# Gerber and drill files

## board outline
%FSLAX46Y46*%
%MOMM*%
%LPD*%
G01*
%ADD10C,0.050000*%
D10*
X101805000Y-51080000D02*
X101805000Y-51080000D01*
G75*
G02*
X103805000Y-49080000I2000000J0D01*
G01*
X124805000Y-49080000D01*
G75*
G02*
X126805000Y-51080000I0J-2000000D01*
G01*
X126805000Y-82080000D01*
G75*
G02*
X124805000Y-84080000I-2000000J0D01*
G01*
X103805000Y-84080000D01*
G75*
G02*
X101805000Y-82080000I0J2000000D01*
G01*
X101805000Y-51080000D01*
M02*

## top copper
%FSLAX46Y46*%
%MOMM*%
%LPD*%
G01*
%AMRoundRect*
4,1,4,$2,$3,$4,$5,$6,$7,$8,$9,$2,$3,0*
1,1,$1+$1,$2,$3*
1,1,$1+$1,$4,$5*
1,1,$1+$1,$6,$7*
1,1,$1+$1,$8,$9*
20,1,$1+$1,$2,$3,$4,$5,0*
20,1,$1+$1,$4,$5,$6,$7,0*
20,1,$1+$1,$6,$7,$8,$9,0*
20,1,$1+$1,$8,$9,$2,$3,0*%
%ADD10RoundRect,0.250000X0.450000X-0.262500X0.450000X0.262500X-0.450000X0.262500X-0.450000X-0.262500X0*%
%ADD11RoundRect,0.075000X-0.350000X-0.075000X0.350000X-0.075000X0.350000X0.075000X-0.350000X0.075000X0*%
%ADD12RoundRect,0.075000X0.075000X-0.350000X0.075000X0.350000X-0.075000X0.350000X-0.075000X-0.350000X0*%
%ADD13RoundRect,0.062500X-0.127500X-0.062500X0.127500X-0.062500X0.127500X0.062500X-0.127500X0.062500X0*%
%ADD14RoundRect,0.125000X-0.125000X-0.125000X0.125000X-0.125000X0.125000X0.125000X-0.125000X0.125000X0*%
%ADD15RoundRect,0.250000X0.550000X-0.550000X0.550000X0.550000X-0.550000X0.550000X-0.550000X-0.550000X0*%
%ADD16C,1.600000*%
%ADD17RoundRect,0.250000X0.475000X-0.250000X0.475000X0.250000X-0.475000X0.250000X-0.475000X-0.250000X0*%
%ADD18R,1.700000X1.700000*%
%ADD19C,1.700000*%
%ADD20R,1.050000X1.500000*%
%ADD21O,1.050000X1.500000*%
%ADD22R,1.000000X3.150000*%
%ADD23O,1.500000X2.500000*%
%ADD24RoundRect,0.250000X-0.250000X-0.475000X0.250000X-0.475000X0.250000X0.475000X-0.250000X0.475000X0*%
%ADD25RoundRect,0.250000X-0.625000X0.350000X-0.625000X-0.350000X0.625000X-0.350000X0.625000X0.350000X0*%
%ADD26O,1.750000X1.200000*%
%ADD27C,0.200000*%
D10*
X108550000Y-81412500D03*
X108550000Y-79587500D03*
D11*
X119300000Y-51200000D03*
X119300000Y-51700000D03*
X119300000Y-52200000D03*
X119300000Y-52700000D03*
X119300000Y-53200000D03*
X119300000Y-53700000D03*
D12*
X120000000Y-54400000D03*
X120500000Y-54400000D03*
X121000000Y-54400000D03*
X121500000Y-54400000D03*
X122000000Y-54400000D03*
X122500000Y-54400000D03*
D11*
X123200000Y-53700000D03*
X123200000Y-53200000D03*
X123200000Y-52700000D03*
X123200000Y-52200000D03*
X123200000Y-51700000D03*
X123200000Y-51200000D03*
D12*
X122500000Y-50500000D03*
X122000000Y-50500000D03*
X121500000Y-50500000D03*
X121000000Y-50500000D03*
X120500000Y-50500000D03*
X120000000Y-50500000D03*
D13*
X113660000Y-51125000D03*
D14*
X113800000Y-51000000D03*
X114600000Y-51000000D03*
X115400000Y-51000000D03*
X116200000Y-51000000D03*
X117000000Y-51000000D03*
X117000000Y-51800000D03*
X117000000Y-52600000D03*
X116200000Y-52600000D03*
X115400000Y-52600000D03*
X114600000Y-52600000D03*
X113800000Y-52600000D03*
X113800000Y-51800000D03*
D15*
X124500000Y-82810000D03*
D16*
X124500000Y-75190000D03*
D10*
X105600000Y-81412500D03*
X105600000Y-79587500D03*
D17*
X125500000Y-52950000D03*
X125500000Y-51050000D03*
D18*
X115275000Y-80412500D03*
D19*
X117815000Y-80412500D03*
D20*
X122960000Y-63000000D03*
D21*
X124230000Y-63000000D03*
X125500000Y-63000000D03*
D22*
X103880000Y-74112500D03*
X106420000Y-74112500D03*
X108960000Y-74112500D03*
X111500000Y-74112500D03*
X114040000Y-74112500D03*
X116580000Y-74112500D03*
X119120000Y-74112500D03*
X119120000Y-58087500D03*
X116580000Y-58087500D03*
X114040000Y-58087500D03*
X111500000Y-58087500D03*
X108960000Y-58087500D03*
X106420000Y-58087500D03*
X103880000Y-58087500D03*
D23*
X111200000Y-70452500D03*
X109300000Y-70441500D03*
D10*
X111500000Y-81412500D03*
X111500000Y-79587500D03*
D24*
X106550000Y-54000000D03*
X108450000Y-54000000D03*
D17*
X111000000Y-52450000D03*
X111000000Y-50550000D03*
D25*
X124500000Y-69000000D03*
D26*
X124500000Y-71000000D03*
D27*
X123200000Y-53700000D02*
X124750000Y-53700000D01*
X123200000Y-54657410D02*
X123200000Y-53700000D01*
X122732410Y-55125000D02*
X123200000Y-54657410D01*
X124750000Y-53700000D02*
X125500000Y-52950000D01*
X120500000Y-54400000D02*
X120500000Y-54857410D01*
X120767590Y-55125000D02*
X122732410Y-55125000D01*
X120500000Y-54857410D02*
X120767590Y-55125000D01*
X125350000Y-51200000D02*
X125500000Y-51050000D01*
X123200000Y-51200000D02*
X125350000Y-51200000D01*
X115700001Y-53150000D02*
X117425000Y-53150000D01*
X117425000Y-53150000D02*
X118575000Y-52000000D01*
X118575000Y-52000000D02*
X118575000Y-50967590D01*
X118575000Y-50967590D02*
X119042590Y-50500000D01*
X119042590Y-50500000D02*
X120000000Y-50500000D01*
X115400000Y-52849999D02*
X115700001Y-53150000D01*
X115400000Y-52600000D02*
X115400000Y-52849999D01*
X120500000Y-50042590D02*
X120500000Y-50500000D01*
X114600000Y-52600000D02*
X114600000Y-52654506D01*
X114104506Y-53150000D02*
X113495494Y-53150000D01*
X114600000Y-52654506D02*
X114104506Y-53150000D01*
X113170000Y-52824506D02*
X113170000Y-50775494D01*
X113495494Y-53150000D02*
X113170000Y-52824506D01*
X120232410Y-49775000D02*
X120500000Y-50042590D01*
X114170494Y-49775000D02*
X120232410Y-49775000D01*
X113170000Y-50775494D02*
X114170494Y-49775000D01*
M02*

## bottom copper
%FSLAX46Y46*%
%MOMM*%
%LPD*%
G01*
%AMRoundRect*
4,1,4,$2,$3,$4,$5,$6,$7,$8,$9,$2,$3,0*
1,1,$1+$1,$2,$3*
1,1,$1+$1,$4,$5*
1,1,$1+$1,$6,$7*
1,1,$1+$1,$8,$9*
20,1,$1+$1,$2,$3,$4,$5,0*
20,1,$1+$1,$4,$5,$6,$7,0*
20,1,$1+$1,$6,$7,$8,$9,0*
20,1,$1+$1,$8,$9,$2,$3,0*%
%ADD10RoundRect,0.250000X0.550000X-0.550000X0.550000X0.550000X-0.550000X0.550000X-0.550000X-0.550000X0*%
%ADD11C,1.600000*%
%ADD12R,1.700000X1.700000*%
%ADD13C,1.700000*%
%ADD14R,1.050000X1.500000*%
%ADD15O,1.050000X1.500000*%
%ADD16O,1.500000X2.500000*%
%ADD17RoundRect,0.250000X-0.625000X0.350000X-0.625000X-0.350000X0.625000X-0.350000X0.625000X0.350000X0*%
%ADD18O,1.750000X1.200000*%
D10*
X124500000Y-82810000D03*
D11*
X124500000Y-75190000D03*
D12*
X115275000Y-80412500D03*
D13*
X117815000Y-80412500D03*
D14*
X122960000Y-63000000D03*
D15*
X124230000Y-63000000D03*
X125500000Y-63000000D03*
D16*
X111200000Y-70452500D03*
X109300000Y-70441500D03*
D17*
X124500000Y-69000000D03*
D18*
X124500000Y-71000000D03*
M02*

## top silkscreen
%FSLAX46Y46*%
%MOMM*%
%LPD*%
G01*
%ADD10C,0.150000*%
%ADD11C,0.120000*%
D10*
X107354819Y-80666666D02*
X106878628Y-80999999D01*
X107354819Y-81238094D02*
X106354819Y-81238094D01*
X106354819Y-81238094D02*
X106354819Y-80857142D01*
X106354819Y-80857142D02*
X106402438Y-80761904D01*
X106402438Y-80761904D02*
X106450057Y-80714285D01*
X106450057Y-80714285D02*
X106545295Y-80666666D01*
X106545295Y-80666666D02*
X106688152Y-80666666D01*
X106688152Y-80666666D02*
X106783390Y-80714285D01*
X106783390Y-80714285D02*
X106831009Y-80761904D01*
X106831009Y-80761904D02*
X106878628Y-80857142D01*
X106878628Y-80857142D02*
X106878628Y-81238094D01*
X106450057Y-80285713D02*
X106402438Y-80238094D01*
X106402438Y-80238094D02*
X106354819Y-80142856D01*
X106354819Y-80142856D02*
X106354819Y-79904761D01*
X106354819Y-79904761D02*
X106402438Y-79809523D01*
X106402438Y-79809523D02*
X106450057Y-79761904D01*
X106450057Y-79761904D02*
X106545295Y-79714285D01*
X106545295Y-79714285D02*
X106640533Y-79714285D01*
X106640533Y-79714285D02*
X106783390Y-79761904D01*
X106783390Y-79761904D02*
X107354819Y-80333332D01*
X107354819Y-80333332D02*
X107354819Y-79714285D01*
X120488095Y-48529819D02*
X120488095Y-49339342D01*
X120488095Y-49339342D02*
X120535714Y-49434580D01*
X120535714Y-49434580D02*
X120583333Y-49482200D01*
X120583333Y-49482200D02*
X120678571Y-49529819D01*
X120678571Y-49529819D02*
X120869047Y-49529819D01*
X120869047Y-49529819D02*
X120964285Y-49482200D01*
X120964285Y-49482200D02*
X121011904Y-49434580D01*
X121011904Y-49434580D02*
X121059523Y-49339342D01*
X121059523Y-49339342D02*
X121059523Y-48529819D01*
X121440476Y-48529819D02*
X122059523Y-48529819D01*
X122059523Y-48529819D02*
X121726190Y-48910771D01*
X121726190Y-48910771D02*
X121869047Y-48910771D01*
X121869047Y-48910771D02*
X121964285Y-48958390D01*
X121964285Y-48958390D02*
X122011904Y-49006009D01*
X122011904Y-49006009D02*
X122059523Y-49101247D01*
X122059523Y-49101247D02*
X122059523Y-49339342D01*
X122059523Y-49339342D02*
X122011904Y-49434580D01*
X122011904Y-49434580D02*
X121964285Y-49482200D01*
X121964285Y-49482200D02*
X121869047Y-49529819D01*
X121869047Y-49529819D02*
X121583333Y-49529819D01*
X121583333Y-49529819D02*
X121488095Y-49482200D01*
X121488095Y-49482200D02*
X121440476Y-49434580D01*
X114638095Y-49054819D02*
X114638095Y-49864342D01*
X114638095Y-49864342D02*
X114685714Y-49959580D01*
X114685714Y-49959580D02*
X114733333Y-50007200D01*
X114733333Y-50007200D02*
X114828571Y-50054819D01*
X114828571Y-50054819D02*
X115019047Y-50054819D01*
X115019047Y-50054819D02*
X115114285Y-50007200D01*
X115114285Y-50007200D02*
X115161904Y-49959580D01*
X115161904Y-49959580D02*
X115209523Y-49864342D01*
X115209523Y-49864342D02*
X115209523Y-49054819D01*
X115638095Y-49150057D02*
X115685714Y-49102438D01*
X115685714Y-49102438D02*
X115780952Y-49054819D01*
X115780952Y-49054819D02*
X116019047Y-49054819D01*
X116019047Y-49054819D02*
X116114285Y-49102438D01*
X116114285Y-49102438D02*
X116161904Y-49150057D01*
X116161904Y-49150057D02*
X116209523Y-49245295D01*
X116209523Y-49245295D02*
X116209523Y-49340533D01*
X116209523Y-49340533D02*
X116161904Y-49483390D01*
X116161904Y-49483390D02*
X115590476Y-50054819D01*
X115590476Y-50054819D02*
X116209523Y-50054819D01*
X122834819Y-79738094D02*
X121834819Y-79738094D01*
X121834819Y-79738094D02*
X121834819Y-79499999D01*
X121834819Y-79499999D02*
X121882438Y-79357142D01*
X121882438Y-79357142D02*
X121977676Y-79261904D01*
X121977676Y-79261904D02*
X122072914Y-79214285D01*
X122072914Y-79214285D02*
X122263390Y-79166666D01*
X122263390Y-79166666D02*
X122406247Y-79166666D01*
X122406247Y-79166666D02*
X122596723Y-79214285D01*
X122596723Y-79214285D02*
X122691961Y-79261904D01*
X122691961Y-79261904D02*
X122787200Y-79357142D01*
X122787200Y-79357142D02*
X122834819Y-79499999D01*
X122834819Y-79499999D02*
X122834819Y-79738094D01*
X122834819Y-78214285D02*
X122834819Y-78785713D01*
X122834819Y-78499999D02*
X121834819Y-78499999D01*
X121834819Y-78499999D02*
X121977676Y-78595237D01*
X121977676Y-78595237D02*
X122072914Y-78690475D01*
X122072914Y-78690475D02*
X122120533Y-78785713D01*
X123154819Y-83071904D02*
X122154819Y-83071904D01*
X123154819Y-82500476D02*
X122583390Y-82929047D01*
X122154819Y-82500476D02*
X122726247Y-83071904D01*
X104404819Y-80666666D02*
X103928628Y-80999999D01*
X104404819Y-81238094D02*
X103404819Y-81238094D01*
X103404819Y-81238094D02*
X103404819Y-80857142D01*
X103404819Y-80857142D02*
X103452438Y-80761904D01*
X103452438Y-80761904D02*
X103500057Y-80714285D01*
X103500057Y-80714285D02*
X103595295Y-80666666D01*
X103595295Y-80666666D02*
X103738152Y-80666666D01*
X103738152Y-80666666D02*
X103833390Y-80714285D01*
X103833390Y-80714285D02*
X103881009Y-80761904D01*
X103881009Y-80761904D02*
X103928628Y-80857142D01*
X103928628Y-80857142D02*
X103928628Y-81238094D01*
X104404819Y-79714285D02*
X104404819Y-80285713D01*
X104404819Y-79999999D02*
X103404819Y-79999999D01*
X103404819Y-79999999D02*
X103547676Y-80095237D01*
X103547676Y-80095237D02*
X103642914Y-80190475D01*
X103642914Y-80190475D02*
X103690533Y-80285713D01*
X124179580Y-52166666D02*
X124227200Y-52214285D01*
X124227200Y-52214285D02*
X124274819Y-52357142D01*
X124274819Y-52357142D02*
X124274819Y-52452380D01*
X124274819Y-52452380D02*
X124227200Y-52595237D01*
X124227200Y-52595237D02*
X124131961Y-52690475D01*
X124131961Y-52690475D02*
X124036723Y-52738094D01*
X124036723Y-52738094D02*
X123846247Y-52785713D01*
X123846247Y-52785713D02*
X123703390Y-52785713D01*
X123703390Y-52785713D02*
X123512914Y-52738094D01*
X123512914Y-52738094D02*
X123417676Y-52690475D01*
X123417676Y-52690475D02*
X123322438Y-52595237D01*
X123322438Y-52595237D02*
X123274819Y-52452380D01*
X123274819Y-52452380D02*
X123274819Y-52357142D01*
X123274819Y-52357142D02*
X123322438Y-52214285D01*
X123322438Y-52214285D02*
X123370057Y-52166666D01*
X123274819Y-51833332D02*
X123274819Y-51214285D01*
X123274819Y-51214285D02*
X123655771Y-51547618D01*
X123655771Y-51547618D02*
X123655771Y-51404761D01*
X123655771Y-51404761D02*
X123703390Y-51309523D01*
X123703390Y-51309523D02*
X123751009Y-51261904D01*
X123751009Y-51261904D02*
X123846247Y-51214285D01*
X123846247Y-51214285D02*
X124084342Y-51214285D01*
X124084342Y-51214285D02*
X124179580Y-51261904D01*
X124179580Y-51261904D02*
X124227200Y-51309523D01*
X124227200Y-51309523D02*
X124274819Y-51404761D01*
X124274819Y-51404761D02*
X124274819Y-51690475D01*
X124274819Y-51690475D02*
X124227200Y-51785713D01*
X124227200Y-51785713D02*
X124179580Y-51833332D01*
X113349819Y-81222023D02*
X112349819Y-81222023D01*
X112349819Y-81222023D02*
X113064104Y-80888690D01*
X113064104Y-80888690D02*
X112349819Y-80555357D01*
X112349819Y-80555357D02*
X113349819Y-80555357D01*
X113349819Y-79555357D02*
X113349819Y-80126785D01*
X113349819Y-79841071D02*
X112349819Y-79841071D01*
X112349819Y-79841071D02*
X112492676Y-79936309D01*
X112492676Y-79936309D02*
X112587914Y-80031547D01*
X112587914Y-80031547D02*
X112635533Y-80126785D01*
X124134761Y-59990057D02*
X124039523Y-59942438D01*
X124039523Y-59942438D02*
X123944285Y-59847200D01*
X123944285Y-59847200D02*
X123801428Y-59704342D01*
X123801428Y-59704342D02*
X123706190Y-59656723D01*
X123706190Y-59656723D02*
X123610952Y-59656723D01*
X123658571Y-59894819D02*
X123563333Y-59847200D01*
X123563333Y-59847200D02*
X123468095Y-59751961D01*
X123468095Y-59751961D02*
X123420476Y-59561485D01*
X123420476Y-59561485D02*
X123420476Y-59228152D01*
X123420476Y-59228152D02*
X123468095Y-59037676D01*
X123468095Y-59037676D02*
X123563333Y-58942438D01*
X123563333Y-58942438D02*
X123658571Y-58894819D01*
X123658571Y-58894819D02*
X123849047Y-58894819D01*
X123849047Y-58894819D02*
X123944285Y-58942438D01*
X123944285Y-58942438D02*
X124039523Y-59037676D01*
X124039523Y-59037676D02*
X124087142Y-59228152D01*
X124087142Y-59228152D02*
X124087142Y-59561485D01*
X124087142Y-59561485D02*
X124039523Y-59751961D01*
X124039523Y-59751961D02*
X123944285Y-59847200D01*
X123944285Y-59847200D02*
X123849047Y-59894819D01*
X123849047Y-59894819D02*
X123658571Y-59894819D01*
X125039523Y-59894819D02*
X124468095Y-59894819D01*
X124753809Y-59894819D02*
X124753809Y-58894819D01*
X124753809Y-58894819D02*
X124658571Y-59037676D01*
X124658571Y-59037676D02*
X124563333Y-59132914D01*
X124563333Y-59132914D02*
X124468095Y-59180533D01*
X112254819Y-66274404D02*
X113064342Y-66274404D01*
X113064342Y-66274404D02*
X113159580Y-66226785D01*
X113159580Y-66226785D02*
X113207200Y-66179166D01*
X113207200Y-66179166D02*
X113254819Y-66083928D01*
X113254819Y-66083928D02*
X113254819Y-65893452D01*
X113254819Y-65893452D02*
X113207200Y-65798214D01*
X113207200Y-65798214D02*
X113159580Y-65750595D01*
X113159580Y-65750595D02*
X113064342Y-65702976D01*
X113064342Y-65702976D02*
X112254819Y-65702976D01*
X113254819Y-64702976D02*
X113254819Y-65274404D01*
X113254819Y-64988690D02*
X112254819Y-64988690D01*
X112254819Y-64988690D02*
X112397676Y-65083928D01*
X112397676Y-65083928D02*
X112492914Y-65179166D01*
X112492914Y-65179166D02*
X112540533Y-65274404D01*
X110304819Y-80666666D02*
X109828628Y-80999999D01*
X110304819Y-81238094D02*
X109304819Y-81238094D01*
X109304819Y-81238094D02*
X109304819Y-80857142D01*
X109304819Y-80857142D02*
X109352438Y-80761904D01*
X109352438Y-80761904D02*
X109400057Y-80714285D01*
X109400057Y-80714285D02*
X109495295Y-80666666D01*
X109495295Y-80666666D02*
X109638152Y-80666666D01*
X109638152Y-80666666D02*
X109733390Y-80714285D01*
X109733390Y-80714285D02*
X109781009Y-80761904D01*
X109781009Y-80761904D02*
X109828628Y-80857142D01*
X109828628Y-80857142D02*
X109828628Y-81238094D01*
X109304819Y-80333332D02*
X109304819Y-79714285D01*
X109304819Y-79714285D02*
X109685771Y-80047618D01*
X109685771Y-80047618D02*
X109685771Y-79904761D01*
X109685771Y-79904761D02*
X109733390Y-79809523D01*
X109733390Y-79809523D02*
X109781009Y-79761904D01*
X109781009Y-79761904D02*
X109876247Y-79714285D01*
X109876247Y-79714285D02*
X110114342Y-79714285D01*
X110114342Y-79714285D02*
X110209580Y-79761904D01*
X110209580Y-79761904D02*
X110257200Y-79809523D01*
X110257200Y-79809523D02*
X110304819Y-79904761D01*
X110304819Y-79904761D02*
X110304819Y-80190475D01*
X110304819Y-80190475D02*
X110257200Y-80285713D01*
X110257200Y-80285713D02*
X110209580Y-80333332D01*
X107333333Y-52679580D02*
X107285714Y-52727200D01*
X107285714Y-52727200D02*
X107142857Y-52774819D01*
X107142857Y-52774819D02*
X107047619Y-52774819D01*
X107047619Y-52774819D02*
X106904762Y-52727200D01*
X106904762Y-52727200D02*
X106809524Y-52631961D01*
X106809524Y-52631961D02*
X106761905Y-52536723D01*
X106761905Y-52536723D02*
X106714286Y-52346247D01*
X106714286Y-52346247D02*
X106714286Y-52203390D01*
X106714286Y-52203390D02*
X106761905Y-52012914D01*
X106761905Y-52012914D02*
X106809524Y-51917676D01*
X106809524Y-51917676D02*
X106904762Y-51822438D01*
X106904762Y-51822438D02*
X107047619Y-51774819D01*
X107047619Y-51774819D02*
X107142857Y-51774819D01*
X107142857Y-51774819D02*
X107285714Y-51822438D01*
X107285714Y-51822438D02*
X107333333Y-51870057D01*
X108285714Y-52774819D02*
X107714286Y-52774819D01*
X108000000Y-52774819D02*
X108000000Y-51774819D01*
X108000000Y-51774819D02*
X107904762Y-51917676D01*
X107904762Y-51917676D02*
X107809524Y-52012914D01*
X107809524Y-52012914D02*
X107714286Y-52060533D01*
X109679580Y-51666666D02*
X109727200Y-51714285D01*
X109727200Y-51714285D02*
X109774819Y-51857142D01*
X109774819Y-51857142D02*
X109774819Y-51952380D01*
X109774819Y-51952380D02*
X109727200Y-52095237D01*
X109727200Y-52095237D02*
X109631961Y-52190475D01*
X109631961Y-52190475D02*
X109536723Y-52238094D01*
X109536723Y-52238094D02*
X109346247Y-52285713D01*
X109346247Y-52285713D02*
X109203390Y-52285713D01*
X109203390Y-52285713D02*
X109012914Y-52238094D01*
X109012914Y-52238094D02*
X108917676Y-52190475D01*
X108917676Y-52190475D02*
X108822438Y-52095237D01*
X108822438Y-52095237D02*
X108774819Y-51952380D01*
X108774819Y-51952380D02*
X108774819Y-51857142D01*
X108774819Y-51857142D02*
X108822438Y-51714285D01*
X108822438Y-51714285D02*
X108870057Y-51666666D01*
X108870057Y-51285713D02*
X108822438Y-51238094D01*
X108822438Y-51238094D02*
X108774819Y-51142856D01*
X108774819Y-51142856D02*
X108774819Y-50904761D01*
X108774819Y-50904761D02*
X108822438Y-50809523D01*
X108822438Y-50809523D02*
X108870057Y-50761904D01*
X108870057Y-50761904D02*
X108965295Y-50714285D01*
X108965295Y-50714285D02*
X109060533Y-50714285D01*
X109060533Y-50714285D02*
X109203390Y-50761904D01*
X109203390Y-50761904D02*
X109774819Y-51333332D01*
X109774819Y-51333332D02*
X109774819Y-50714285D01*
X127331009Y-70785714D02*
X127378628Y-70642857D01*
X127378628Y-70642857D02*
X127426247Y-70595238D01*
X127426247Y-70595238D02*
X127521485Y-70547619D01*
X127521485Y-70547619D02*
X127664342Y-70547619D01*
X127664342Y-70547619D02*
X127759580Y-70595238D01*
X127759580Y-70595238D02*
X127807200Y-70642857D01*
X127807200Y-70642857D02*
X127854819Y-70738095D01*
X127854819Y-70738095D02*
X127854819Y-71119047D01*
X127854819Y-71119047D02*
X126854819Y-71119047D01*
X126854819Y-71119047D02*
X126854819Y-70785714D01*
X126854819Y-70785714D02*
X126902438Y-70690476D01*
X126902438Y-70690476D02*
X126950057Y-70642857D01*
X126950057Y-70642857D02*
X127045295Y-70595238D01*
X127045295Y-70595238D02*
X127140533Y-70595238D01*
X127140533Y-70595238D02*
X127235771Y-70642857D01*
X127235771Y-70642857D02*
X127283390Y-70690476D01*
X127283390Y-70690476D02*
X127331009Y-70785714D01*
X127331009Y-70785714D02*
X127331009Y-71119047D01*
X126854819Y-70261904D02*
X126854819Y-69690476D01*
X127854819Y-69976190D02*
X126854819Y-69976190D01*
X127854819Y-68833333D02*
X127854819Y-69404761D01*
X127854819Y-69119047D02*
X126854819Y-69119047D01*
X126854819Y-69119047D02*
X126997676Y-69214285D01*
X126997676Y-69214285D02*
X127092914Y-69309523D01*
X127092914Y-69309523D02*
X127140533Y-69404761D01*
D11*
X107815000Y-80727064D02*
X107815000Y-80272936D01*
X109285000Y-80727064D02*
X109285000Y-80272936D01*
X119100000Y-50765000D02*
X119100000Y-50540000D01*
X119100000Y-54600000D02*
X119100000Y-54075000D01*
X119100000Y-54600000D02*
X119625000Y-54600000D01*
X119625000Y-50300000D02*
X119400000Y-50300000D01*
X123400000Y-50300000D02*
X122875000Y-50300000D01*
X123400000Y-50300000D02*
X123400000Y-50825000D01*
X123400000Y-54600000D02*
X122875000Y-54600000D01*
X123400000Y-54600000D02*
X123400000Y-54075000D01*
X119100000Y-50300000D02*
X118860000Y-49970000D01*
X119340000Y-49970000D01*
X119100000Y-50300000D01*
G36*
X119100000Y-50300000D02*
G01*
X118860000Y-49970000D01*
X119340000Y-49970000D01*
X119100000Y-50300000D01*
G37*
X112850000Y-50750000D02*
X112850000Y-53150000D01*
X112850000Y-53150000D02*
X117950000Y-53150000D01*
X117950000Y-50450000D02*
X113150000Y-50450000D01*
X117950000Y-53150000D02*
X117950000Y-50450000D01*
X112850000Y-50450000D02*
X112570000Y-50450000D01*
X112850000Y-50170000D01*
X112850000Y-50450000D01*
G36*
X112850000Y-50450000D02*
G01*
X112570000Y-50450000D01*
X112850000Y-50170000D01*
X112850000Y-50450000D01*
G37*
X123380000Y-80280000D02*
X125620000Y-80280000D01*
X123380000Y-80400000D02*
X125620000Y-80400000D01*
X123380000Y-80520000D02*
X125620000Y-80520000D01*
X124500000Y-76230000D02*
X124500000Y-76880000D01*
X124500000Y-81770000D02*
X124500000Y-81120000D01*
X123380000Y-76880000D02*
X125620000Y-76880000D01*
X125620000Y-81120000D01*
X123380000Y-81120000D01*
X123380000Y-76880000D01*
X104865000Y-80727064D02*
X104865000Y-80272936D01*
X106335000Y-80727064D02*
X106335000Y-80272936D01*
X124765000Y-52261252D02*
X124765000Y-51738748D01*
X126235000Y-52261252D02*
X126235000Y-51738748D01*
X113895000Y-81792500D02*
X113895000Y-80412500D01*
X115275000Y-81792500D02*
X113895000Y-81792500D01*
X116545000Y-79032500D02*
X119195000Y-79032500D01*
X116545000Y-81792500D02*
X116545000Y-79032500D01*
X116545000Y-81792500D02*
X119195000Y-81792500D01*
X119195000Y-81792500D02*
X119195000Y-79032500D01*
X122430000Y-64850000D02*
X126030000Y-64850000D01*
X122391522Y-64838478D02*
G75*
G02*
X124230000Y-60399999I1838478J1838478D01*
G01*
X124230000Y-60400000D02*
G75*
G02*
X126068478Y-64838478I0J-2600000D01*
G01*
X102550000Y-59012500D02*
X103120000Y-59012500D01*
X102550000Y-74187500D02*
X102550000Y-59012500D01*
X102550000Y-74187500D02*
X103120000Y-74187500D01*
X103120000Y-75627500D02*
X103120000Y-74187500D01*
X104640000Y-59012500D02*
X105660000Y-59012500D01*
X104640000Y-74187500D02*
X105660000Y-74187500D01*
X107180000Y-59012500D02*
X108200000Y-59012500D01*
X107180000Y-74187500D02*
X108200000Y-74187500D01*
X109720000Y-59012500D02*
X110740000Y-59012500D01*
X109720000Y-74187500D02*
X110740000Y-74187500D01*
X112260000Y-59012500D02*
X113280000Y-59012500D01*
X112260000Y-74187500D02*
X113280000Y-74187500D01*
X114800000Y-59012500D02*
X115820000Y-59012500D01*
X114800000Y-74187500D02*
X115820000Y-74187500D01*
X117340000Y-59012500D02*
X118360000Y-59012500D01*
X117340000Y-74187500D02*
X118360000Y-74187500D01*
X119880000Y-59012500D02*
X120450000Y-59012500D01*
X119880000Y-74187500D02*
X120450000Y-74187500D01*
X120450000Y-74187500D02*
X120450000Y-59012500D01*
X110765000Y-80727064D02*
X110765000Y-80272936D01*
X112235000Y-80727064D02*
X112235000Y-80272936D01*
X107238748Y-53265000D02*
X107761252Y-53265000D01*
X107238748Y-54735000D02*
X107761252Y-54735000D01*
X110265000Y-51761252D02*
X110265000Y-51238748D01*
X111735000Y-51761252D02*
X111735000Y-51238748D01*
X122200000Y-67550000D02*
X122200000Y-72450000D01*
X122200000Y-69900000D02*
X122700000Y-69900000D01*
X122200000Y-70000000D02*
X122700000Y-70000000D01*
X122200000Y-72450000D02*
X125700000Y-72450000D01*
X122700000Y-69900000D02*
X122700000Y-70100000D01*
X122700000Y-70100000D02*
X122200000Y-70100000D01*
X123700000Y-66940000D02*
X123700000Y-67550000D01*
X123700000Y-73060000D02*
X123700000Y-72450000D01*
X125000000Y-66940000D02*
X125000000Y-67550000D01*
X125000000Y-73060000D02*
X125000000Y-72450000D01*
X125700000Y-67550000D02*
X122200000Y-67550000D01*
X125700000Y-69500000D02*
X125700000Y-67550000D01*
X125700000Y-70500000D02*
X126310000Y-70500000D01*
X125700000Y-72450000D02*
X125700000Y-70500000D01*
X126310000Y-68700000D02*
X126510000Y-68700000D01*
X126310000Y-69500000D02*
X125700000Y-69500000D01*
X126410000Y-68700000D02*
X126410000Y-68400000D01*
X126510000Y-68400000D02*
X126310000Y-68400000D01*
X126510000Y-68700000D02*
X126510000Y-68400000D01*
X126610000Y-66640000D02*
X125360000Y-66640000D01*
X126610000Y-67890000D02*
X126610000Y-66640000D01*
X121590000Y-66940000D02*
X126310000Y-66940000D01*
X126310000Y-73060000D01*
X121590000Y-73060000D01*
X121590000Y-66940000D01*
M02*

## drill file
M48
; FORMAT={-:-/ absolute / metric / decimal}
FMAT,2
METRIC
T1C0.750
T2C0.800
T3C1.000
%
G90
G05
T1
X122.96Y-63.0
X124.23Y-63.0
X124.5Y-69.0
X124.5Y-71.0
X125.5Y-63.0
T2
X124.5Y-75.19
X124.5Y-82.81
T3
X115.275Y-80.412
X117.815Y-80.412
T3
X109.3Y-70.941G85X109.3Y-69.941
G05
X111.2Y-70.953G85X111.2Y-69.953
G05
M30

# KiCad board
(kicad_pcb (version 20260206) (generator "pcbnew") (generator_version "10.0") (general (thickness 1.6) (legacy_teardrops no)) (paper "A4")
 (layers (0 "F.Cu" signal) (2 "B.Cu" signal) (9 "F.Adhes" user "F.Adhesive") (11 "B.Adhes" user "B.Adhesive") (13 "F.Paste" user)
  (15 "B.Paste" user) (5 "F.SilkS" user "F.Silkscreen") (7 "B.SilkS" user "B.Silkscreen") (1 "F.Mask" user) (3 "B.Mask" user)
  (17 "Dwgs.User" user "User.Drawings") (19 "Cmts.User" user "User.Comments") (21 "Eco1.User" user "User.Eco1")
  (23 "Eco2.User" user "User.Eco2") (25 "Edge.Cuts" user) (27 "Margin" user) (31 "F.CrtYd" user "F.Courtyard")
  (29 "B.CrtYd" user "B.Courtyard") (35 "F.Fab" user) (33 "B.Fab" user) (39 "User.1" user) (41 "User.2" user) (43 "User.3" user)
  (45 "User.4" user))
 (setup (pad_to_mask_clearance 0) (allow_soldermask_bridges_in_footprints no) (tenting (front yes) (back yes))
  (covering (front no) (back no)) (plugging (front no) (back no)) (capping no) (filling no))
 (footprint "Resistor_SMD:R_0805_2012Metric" (layer "F.Cu") (at 108.55 80.5 90)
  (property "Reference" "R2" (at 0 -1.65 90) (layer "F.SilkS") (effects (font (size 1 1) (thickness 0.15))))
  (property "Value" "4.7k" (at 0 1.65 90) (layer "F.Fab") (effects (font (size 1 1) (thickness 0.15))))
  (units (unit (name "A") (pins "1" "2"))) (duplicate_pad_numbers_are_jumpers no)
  (fp_line (start -0.227064 -0.735) (end 0.227064 -0.735) (stroke (width 0.12) (type solid)) (layer "F.SilkS"))
  (fp_line (start -0.227064 0.735) (end 0.227064 0.735) (stroke (width 0.12) (type solid)) (layer "F.SilkS"))
  (pad "1" smd roundrect (at -0.9125 0 90) (size 1.025 1.4) (layers "F.Cu" "F.Mask" "F.Paste") (roundrect_rratio 0.243902) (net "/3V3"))
  (pad "2" smd roundrect (at 0.9125 0 90) (size 1.025 1.4) (layers "F.Cu" "F.Mask" "F.Paste") (roundrect_rratio 0.243902) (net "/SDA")))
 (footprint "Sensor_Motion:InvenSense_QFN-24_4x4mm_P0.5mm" (layer "F.Cu") (at 121.25 52.45)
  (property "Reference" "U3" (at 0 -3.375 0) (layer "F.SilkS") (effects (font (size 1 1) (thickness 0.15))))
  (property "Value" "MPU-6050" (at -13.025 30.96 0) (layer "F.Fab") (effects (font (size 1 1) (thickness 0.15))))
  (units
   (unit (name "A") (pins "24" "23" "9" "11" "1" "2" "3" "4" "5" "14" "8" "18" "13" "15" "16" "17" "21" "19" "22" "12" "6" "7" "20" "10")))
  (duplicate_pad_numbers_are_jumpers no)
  (fp_line (start -2.15 -1.685) (end -2.15 -1.91) (stroke (width 0.12) (type solid)) (layer "F.SilkS"))
  (fp_line (start -2.15 2.15) (end -2.15 1.625) (stroke (width 0.12) (type solid)) (layer "F.SilkS"))
  (fp_line (start -2.15 2.15) (end -1.625 2.15) (stroke (width 0.12) (type solid)) (layer "F.SilkS"))
  (fp_line (start -1.625 -2.15) (end -1.85 -2.15) (stroke (width 0.12) (type solid)) (layer "F.SilkS"))
  (fp_line (start 2.15 -2.15) (end 1.625 -2.15) (stroke (width 0.12) (type solid)) (layer "F.SilkS"))
  (fp_line (start 2.15 -2.15) (end 2.15 -1.625) (stroke (width 0.12) (type solid)) (layer "F.SilkS"))
  (fp_line (start 2.15 2.15) (end 1.625 2.15) (stroke (width 0.12) (type solid)) (layer "F.SilkS"))
  (fp_line (start 2.15 2.15) (end 2.15 1.625) (stroke (width 0.12) (type solid)) (layer "F.SilkS"))
  (fp_poly
   (pts (xy -2.15 -2.15) (xy -2.39 -2.48) (xy -1.91 -2.48) (xy -2.15 -2.15)) (stroke (width 0.12) (type solid)) (fill yes) (layer "F.SilkS"))
  (pad "1" smd roundrect (at -1.95 -1.25) (size 0.85 0.3) (layers "F.Cu" "F.Mask" "F.Paste") (roundrect_rratio 0.25)
   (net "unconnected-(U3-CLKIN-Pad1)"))
  (pad "2" smd roundrect (at -1.95 -0.75) (size 0.85 0.3) (layers "F.Cu" "F.Mask" "F.Paste") (roundrect_rratio 0.25)
   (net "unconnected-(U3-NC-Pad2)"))
  (pad "3" smd roundrect (at -1.95 -0.25) (size 0.85 0.3) (layers "F.Cu" "F.Mask" "F.Paste") (roundrect_rratio 0.25)
   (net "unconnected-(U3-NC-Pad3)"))
  (pad "4" smd roundrect (at -1.95 0.25) (size 0.85 0.3) (layers "F.Cu" "F.Mask" "F.Paste") (roundrect_rratio 0.25)
   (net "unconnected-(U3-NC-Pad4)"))
  (pad "5" smd roundrect (at -1.95 0.75) (size 0.85 0.3) (layers "F.Cu" "F.Mask" "F.Paste") (roundrect_rratio 0.25)
   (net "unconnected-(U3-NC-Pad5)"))
  (pad "6" smd roundrect (at -1.95 1.25) (size 0.85 0.3) (layers "F.Cu" "F.Mask" "F.Paste") (roundrect_rratio 0.25)
   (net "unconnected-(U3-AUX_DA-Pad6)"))
  (pad "7" smd roundrect (at -1.25 1.95 90) (size 0.85 0.3) (layers "F.Cu" "F.Mask" "F.Paste") (roundrect_rratio 0.25)
   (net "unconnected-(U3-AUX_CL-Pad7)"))
  (pad "8" smd roundrect (at -0.75 1.95 90) (size 0.85 0.3) (layers "F.Cu" "F.Mask" "F.Paste") (roundrect_rratio 0.25) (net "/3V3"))
  (pad "9" smd roundrect (at -0.25 1.95 90) (size 0.85 0.3) (layers "F.Cu" "F.Mask" "F.Paste") (roundrect_rratio 0.25) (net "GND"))
  (pad "10" smd roundrect (at 0.25 1.95 90) (size 0.85 0.3) (layers "F.Cu" "F.Mask" "F.Paste") (roundrect_rratio 0.25)
   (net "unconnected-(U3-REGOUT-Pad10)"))
  (pad "11" smd roundrect (at 0.75 1.95 90) (size 0.85 0.3) (layers "F.Cu" "F.Mask" "F.Paste") (roundrect_rratio 0.25)
   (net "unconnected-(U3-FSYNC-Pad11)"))
  (pad "12" smd roundrect (at 1.25 1.95 90) (size 0.85 0.3) (layers "F.Cu" "F.Mask" "F.Paste") (roundrect_rratio 0.25)
   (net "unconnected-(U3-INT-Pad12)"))
  (pad "13" smd roundrect (at 1.95 1.25) (size 0.85 0.3) (layers "F.Cu" "F.Mask" "F.Paste") (roundrect_rratio 0.25) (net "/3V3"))
  (pad "14" smd roundrect (at 1.95 0.75) (size 0.85 0.3) (layers "F.Cu" "F.Mask" "F.Paste") (roundrect_rratio 0.25)
   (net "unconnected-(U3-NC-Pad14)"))
  (pad "15" smd roundrect (at 1.95 0.25) (size 0.85 0.3) (layers "F.Cu" "F.Mask" "F.Paste") (roundrect_rratio 0.25)
   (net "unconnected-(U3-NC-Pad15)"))
  (pad "16" smd roundrect (at 1.95 -0.25) (size 0.85 0.3) (layers "F.Cu" "F.Mask" "F.Paste") (roundrect_rratio 0.25)
   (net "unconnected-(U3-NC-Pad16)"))
  (pad "17" smd roundrect (at 1.95 -0.75) (size 0.85 0.3) (layers "F.Cu" "F.Mask" "F.Paste") (roundrect_rratio 0.25)
   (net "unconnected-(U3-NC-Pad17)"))
  (pad "18" smd roundrect (at 1.95 -1.25) (size 0.85 0.3) (layers "F.Cu" "F.Mask" "F.Paste") (roundrect_rratio 0.25) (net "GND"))
  (pad "19" smd roundrect (at 1.25 -1.95 90) (size 0.85 0.3) (layers "F.Cu" "F.Mask" "F.Paste") (roundrect_rratio 0.25)
   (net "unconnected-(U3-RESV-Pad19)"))
  (pad "20" smd roundrect (at 0.75 -1.95 90) (size 0.85 0.3) (layers "F.Cu" "F.Mask" "F.Paste") (roundrect_rratio 0.25)
   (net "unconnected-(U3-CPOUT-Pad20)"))
  (pad "21" smd roundrect (at 0.25 -1.95 90) (size 0.85 0.3) (layers "F.Cu" "F.Mask" "F.Paste") (roundrect_rratio 0.25)
   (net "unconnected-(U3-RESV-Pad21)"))
  (pad "22" smd roundrect (at -0.25 -1.95 90) (size 0.85 0.3) (layers "F.Cu" "F.Mask" "F.Paste") (roundrect_rratio 0.25)
   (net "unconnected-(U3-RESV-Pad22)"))
  (pad "23" smd roundrect (at -0.75 -1.95 90) (size 0.85 0.3) (layers "F.Cu" "F.Mask" "F.Paste") (roundrect_rratio 0.25) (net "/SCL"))
  (pad "24" smd roundrect (at -1.25 -1.95 90) (size 0.85 0.3) (layers "F.Cu" "F.Mask" "F.Paste") (roundrect_rratio 0.25) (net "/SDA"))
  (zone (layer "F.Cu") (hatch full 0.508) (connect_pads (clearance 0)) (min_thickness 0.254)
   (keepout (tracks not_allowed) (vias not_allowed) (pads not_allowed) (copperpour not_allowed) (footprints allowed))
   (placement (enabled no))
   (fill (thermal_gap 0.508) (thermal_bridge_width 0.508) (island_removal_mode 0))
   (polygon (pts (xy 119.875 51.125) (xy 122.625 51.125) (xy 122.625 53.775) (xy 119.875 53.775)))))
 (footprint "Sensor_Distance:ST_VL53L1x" (layer "F.Cu") (at 115.4 51.8)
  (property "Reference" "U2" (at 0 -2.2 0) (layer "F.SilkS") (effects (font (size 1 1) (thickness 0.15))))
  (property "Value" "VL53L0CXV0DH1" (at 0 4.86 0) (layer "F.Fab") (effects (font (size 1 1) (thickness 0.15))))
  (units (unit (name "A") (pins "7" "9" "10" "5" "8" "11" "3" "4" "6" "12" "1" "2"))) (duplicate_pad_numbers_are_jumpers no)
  (fp_line (start -2.55 -1.05) (end -2.55 1.35) (stroke (width 0.12) (type solid)) (layer "F.SilkS"))
  (fp_line (start -2.55 1.35) (end 2.55 1.35) (stroke (width 0.12) (type solid)) (layer "F.SilkS"))
  (fp_line (start 2.55 -1.35) (end -2.25 -1.35) (stroke (width 0.12) (type solid)) (layer "F.SilkS"))
  (fp_line (start 2.55 1.35) (end 2.55 -1.35) (stroke (width 0.12) (type solid)) (layer "F.SilkS"))
  (fp_poly
   (pts (xy -2.55 -1.35) (xy -2.83 -1.35) (xy -2.55 -1.63) (xy -2.55 -1.35)) (stroke (width 0.12) (type solid)) (fill yes) (layer "F.SilkS"))
  (pad "1" smd roundrect (at -1.74 -0.675) (size 0.38 0.25) (layers "F.Cu" "F.Mask" "F.Paste") (roundrect_rratio 0.25) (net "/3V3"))
  (pad "1" smd roundrect (at -1.6 -0.8) (size 0.5 0.5) (layers "F.Cu" "F.Mask" "F.Paste") (roundrect_rratio 0.25) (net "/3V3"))
  (pad "2" smd roundrect (at -0.8 -0.8) (size 0.5 0.5) (layers "F.Cu" "F.Mask" "F.Paste") (roundrect_rratio 0.25) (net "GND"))
  (pad "3" smd roundrect (at 0 -0.8) (size 0.5 0.5) (layers "F.Cu" "F.Mask" "F.Paste") (roundrect_rratio 0.25) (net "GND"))
  (pad "4" smd roundrect (at 0.8 -0.8) (size 0.5 0.5) (layers "F.Cu" "F.Mask" "F.Paste") (roundrect_rratio 0.25) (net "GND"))
  (pad "5" smd roundrect (at 1.6 -0.8) (size 0.5 0.5) (layers "F.Cu" "F.Mask" "F.Paste") (roundrect_rratio 0.25) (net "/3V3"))
  (pad "6" smd roundrect (at 1.6 0) (size 0.5 0.5) (layers "F.Cu" "F.Mask" "F.Paste") (roundrect_rratio 0.25) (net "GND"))
  (pad "7" smd roundrect (at 1.6 0.8) (size 0.5 0.5) (layers "F.Cu" "F.Mask" "F.Paste") (roundrect_rratio 0.25)
   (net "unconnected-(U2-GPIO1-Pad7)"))
  (pad "8" smd roundrect (at 0.8 0.8) (size 0.5 0.5) (layers "F.Cu" "F.Mask" "F.Paste") (roundrect_rratio 0.25)
   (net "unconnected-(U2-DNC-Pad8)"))
  (pad "9" smd roundrect (at 0 0.8) (size 0.5 0.5) (layers "F.Cu" "F.Mask" "F.Paste") (roundrect_rratio 0.25) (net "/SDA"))
  (pad "10" smd roundrect (at -0.8 0.8) (size 0.5 0.5) (layers "F.Cu" "F.Mask" "F.Paste") (roundrect_rratio 0.25) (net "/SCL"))
  (pad "11" smd roundrect (at -1.6 0.8) (size 0.5 0.5) (layers "F.Cu" "F.Mask" "F.Paste") (roundrect_rratio 0.25) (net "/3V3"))
  (pad "12" smd roundrect (at -1.6 0) (size 0.5 0.5) (layers "F.Cu" "F.Mask" "F.Paste") (roundrect_rratio 0.25) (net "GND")))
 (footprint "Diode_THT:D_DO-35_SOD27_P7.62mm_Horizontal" (layer "F.Cu") (at 124.5 82.81 90)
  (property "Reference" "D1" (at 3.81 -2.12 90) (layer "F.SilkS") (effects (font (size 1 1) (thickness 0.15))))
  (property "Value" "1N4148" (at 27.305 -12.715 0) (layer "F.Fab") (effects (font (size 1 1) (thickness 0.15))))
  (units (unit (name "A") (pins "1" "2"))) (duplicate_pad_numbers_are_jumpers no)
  (fp_line (start 2.53 -1.12) (end 2.53 1.12) (stroke (width 0.12) (type solid)) (layer "F.SilkS"))
  (fp_line (start 2.41 -1.12) (end 2.41 1.12) (stroke (width 0.12) (type solid)) (layer "F.SilkS"))
  (fp_line (start 2.29 -1.12) (end 2.29 1.12) (stroke (width 0.12) (type solid)) (layer "F.SilkS"))
  (fp_line (start 6.58 0) (end 5.93 0) (stroke (width 0.12) (type solid)) (layer "F.SilkS"))
  (fp_line (start 1.04 0) (end 1.69 0) (stroke (width 0.12) (type solid)) (layer "F.SilkS"))
  (fp_rect (start 1.69 -1.12) (end 5.93 1.12) (stroke (width 0.12) (type solid)) (fill no) (layer "F.SilkS"))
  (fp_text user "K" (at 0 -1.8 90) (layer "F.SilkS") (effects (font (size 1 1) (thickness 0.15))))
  (pad "1" thru_hole roundrect (at 0 0 90) (size 1.6 1.6) (drill 0.8) (layers "*.Cu" "*.Mask") (remove_unused_layers no)
   (roundrect_rratio 0.15625) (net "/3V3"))
  (pad "2" thru_hole circle (at 7.62 0 90) (size 1.6 1.6) (drill 0.8) (layers "*.Cu" "*.Mask") (remove_unused_layers no) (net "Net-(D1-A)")))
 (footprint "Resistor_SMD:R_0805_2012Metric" (layer "F.Cu") (at 105.6 80.5 90)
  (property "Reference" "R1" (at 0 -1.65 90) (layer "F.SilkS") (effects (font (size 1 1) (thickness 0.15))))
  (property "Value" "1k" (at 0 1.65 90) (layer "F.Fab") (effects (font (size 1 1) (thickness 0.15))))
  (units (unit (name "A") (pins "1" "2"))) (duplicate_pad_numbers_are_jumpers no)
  (fp_line (start -0.227064 -0.735) (end 0.227064 -0.735) (stroke (width 0.12) (type solid)) (layer "F.SilkS"))
  (fp_line (start -0.227064 0.735) (end 0.227064 0.735) (stroke (width 0.12) (type solid)) (layer "F.SilkS"))
  (pad "1" smd roundrect (at -0.9125 0 90) (size 1.025 1.4) (layers "F.Cu" "F.Mask" "F.Paste") (roundrect_rratio 0.243902)
   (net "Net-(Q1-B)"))
  (pad "2" smd roundrect (at 0.9125 0 90) (size 1.025 1.4) (layers "F.Cu" "F.Mask" "F.Paste") (roundrect_rratio 0.243902)
   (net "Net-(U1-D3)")))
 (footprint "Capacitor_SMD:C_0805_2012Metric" (layer "F.Cu") (at 125.5 52 90)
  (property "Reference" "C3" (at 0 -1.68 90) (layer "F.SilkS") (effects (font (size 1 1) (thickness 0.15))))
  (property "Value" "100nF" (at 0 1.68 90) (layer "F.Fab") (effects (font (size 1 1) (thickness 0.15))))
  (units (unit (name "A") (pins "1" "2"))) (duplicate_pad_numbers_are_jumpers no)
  (fp_line (start -0.261252 -0.735) (end 0.261252 -0.735) (stroke (width 0.12) (type solid)) (layer "F.SilkS"))
  (fp_line (start -0.261252 0.735) (end 0.261252 0.735) (stroke (width 0.12) (type solid)) (layer "F.SilkS"))
  (pad "1" smd roundrect (at -0.95 0 90) (size 1 1.45) (layers "F.Cu" "F.Mask" "F.Paste") (roundrect_rratio 0.25) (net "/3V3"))
  (pad "2" smd roundrect (at 0.95 0 90) (size 1 1.45) (layers "F.Cu" "F.Mask" "F.Paste") (roundrect_rratio 0.25) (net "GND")))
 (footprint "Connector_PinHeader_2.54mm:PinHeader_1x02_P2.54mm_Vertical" (layer "F.Cu") (at 115.275 80.4125 90)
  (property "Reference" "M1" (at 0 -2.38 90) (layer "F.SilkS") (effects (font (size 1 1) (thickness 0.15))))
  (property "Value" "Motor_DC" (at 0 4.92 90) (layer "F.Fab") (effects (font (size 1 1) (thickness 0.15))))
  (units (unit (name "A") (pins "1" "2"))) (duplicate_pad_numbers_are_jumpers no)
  (fp_line (start -1.38 -1.38) (end 0 -1.38) (stroke (width 0.12) (type solid)) (layer "F.SilkS"))
  (fp_line (start -1.38 0) (end -1.38 -1.38) (stroke (width 0.12) (type solid)) (layer "F.SilkS"))
  (fp_line (start 1.38 1.27) (end 1.38 3.92) (stroke (width 0.12) (type solid)) (layer "F.SilkS"))
  (fp_line (start -1.38 1.27) (end 1.38 1.27) (stroke (width 0.12) (type solid)) (layer "F.SilkS"))
  (fp_line (start -1.38 1.27) (end -1.38 3.92) (stroke (width 0.12) (type solid)) (layer "F.SilkS"))
  (fp_line (start -1.38 3.92) (end 1.38 3.92) (stroke (width 0.12) (type solid)) (layer "F.SilkS"))
  (pad "1" thru_hole rect (at 0 0 90) (size 1.7 1.7) (drill 1) (layers "*.Cu" "*.Mask") (remove_unused_layers no) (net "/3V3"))
  (pad "2" thru_hole circle (at 0 2.54 90) (size 1.7 1.7) (drill 1) (layers "*.Cu" "*.Mask") (remove_unused_layers no) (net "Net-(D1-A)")))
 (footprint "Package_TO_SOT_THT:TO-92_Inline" (layer "F.Cu") (at 122.96 63)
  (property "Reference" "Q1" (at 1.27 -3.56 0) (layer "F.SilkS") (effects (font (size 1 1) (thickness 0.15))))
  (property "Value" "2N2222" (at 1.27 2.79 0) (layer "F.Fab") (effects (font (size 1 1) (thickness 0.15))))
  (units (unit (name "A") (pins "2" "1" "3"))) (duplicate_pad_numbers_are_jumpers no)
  (fp_line (start -0.53 1.85) (end 3.07 1.85) (stroke (width 0.12) (type solid)) (layer "F.SilkS"))
  (fp_arc (start -0.568478 1.838478) (mid -1.132087 -0.994977) (end 1.27 -2.6) (stroke (width 0.12) (type solid)) (layer "F.SilkS"))
  (fp_arc (start 1.27 -2.6) (mid 3.672087 -0.994977) (end 3.108478 1.838478) (stroke (width 0.12) (type solid)) (layer "F.SilkS"))
  (pad "1" thru_hole rect (at 0 0) (size 1.05 1.5) (drill 0.75) (layers "*.Cu" "*.Mask") (remove_unused_layers no) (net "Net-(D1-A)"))
  (pad "2" thru_hole oval (at 1.27 0) (size 1.05 1.5) (drill 0.75) (layers "*.Cu" "*.Mask") (remove_unused_layers no) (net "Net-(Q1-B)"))
  (pad "3" thru_hole oval (at 2.54 0) (size 1.05 1.5) (drill 0.75) (layers "*.Cu" "*.Mask") (remove_unused_layers no) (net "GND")))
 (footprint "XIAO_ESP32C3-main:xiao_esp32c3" (layer "F.Cu") (at 113.3 65.5125 90)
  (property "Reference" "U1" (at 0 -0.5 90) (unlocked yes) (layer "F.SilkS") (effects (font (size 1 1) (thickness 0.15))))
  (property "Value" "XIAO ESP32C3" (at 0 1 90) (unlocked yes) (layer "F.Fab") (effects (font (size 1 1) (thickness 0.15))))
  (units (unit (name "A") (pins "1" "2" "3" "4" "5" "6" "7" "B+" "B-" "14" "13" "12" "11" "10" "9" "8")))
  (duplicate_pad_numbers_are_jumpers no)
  (fp_line (start 6.5 -10.75) (end 6.5 -10.18) (stroke (width 0.12) (type solid)) (layer "F.SilkS"))
  (fp_line (start -8.675 -10.75) (end 6.5 -10.75) (stroke (width 0.12) (type solid)) (layer "F.SilkS"))
  (fp_line (start -8.675 -10.75) (end -8.675 -10.18) (stroke (width 0.12) (type solid)) (layer "F.SilkS"))
  (fp_line (start -10.115 -10.18) (end -8.675 -10.18) (stroke (width 0.12) (type solid)) (layer "F.SilkS"))
  (fp_line (start 6.5 -8.66) (end 6.5 -7.64) (stroke (width 0.12) (type solid)) (layer "F.SilkS"))
  (fp_line (start -8.675 -8.66) (end -8.675 -7.64) (stroke (width 0.12) (type solid)) (layer "F.SilkS"))
  (fp_line (start 6.5 -6.12) (end 6.5 -5.1) (stroke (width 0.12) (type solid)) (layer "F.SilkS"))
  (fp_line (start -8.675 -6.12) (end -8.675 -5.1) (stroke (width 0.12) (type solid)) (layer "F.SilkS"))
  (fp_line (start 6.5 -3.58) (end 6.5 -2.56) (stroke (width 0.12) (type solid)) (layer "F.SilkS"))
  (fp_line (start -8.675 -3.58) (end -8.675 -2.56) (stroke (width 0.12) (type solid)) (layer "F.SilkS"))
  (fp_line (start 6.5 -1.04) (end 6.5 -0.02) (stroke (width 0.12) (type solid)) (layer "F.SilkS"))
  (fp_line (start -8.675 -1.04) (end -8.675 -0.02) (stroke (width 0.12) (type solid)) (layer "F.SilkS"))
  (fp_line (start 6.5 1.5) (end 6.5 2.52) (stroke (width 0.12) (type solid)) (layer "F.SilkS"))
  (fp_line (start -8.675 1.5) (end -8.675 2.52) (stroke (width 0.12) (type solid)) (layer "F.SilkS"))
  (fp_line (start 6.5 4.04) (end 6.5 5.06) (stroke (width 0.12) (type solid)) (layer "F.SilkS"))
  (fp_line (start -8.675 4.04) (end -8.675 5.06) (stroke (width 0.12) (type solid)) (layer "F.SilkS"))
  (fp_line (start 6.5 6.58) (end 6.5 7.15) (stroke (width 0.12) (type solid)) (layer "F.SilkS"))
  (fp_line (start -8.675 6.58) (end -8.675 7.15) (stroke (width 0.12) (type solid)) (layer "F.SilkS"))
  (fp_line (start -8.675 7.15) (end 6.5 7.15) (stroke (width 0.12) (type solid)) (layer "F.SilkS"))
  (pad "1" smd rect (at -8.6 -9.42 90) (size 3.15 1) (layers "F.Cu" "F.Mask" "F.Paste") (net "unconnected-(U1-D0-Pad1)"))
  (pad "2" smd rect (at -8.6 -6.88 90) (size 3.15 1) (layers "F.Cu" "F.Mask" "F.Paste") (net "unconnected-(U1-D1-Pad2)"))
  (pad "3" smd rect (at -8.6 -4.34 90) (size 3.15 1) (layers "F.Cu" "F.Mask" "F.Paste") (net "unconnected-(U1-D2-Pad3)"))
  (pad "4" smd rect (at -8.6 -1.8 90) (size 3.15 1) (layers "F.Cu" "F.Mask" "F.Paste") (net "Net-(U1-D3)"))
  (pad "5" smd rect (at -8.6 0.74 90) (size 3.15 1) (layers "F.Cu" "F.Mask" "F.Paste") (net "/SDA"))
  (pad "6" smd rect (at -8.6 3.28 90) (size 3.15 1) (layers "F.Cu" "F.Mask" "F.Paste") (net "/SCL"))
  (pad "7" smd rect (at -8.6 5.82 90) (size 3.15 1) (layers "F.Cu" "F.Mask" "F.Paste") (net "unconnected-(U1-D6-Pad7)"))
  (pad "8" smd rect (at 7.425 5.82 90) (size 3.15 1) (layers "F.Cu" "F.Mask" "F.Paste") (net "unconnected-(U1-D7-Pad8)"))
  (pad "9" smd rect (at 7.425 3.28 90) (size 3.15 1) (layers "F.Cu" "F.Mask" "F.Paste") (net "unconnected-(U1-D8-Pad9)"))
  (pad "10" smd rect (at 7.425 0.74 90) (size 3.15 1) (layers "F.Cu" "F.Mask" "F.Paste") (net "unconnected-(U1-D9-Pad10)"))
  (pad "11" smd rect (at 7.425 -1.8 90) (size 3.15 1) (layers "F.Cu" "F.Mask" "F.Paste") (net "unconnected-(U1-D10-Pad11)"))
  (pad "12" smd rect (at 7.425 -4.34 90) (size 3.15 1) (layers "F.Cu" "F.Mask" "F.Paste") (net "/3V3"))
  (pad "13" smd rect (at 7.425 -6.88 90) (size 3.15 1) (layers "F.Cu" "F.Mask" "F.Paste") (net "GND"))
  (pad "14" smd rect (at 7.425 -9.42 90) (size 3.15 1) (layers "F.Cu" "F.Mask" "F.Paste") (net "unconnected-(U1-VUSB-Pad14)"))
  (pad "B+" thru_hole oval (at -4.94 -2.1 90) (size 2.5 1.5) (drill oval 2 1) (layers "*.Cu" "*.Mask") (remove_unused_layers no)
   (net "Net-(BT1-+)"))
  (pad "B-" thru_hole oval (at -4.929 -4 90) (size 2.5 1.5) (drill oval 2 1) (layers "*.Cu" "*.Mask") (remove_unused_layers no)
   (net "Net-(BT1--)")))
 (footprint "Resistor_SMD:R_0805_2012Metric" (layer "F.Cu") (at 111.5 80.5 90)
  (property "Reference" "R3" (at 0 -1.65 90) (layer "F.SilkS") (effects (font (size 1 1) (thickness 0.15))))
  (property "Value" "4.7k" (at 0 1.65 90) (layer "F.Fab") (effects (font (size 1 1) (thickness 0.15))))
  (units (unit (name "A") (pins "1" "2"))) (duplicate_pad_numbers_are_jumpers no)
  (fp_line (start -0.227064 -0.735) (end 0.227064 -0.735) (stroke (width 0.12) (type solid)) (layer "F.SilkS"))
  (fp_line (start -0.227064 0.735) (end 0.227064 0.735) (stroke (width 0.12) (type solid)) (layer "F.SilkS"))
  (pad "1" smd roundrect (at -0.9125 0 90) (size 1.025 1.4) (layers "F.Cu" "F.Mask" "F.Paste") (roundrect_rratio 0.243902) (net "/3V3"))
  (pad "2" smd roundrect (at 0.9125 0 90) (size 1.025 1.4) (layers "F.Cu" "F.Mask" "F.Paste") (roundrect_rratio 0.243902) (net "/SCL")))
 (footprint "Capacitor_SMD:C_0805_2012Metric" (layer "F.Cu") (at 107.5 54)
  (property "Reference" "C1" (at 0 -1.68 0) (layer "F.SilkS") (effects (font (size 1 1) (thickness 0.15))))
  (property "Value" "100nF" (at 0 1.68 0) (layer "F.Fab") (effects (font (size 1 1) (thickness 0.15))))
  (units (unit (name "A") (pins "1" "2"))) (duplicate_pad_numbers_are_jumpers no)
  (fp_line (start -0.261252 -0.735) (end 0.261252 -0.735) (stroke (width 0.12) (type solid)) (layer "F.SilkS"))
  (fp_line (start -0.261252 0.735) (end 0.261252 0.735) (stroke (width 0.12) (type solid)) (layer "F.SilkS"))
  (pad "1" smd roundrect (at -0.95 0) (size 1 1.45) (layers "F.Cu" "F.Mask" "F.Paste") (roundrect_rratio 0.25) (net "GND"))
  (pad "2" smd roundrect (at 0.95 0) (size 1 1.45) (layers "F.Cu" "F.Mask" "F.Paste") (roundrect_rratio 0.25) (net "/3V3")))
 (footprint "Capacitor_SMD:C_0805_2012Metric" (layer "F.Cu") (at 111 51.5 90)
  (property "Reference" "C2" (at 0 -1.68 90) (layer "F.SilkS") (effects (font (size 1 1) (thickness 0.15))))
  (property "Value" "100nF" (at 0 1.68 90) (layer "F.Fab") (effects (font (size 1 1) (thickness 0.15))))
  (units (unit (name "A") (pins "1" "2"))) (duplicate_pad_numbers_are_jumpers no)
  (fp_line (start -0.261252 -0.735) (end 0.261252 -0.735) (stroke (width 0.12) (type solid)) (layer "F.SilkS"))
  (fp_line (start -0.261252 0.735) (end 0.261252 0.735) (stroke (width 0.12) (type solid)) (layer "F.SilkS"))
  (pad "1" smd roundrect (at -0.95 0 90) (size 1 1.45) (layers "F.Cu" "F.Mask" "F.Paste") (roundrect_rratio 0.25) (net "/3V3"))
  (pad "2" smd roundrect (at 0.95 0 90) (size 1 1.45) (layers "F.Cu" "F.Mask" "F.Paste") (roundrect_rratio 0.25) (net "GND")))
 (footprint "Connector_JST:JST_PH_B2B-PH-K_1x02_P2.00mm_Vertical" (layer "F.Cu") (at 124.5 69 -90)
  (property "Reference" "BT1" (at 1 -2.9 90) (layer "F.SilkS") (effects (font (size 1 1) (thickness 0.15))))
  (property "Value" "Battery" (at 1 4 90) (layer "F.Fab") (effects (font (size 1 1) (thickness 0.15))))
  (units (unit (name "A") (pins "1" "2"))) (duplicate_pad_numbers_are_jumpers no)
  (fp_line (start -1.45 2.3) (end 3.45 2.3) (stroke (width 0.12) (type solid)) (layer "F.SilkS"))
  (fp_line (start 0.9 2.3) (end 0.9 1.8) (stroke (width 0.12) (type solid)) (layer "F.SilkS"))
  (fp_line (start 1 2.3) (end 1 1.8) (stroke (width 0.12) (type solid)) (layer "F.SilkS"))
  (fp_line (start 3.45 2.3) (end 3.45 -1.2) (stroke (width 0.12) (type solid)) (layer "F.SilkS"))
  (fp_line (start 0.9 1.8) (end 1.1 1.8) (stroke (width 0.12) (type solid)) (layer "F.SilkS"))
  (fp_line (start 1.1 1.8) (end 1.1 2.3) (stroke (width 0.12) (type solid)) (layer "F.SilkS"))
  (fp_line (start -2.06 0.8) (end -1.45 0.8) (stroke (width 0.12) (type solid)) (layer "F.SilkS"))
  (fp_line (start 4.06 0.8) (end 3.45 0.8) (stroke (width 0.12) (type solid)) (layer "F.SilkS"))
  (fp_line (start -2.06 -0.5) (end -1.45 -0.5) (stroke (width 0.12) (type solid)) (layer "F.SilkS"))
  (fp_line (start 4.06 -0.5) (end 3.45 -0.5) (stroke (width 0.12) (type solid)) (layer "F.SilkS"))
  (fp_line (start -1.45 -1.2) (end -1.45 2.3) (stroke (width 0.12) (type solid)) (layer "F.SilkS"))
  (fp_line (start 0.5 -1.2) (end -1.45 -1.2) (stroke (width 0.12) (type solid)) (layer "F.SilkS"))
  (fp_line (start 1.5 -1.2) (end 1.5 -1.81) (stroke (width 0.12) (type solid)) (layer "F.SilkS"))
  (fp_line (start 3.45 -1.2) (end 1.5 -1.2) (stroke (width 0.12) (type solid)) (layer "F.SilkS"))
  (fp_line (start -0.3 -1.81) (end -0.3 -2.01) (stroke (width 0.12) (type solid)) (layer "F.SilkS"))
  (fp_line (start 0.5 -1.81) (end 0.5 -1.2) (stroke (width 0.12) (type solid)) (layer "F.SilkS"))
  (fp_line (start -0.3 -1.91) (end -0.6 -1.91) (stroke (width 0.12) (type solid)) (layer "F.SilkS"))
  (fp_line (start -0.6 -2.01) (end -0.6 -1.81) (stroke (width 0.12) (type solid)) (layer "F.SilkS"))
  (fp_line (start -0.3 -2.01) (end -0.6 -2.01) (stroke (width 0.12) (type solid)) (layer "F.SilkS"))
  (fp_line (start -2.36 -2.11) (end -2.36 -0.86) (stroke (width 0.12) (type solid)) (layer "F.SilkS"))
  (fp_line (start -1.11 -2.11) (end -2.36 -2.11) (stroke (width 0.12) (type solid)) (layer "F.SilkS"))
  (fp_rect (start -2.06 -1.81) (end 4.06 2.91) (stroke (width 0.12) (type solid)) (fill no) (layer "F.SilkS"))
  (pad "1" thru_hole roundrect (at 0 0 270) (size 1.2 1.75) (drill 0.75) (layers "*.Cu" "*.Mask") (remove_unused_layers no)
   (roundrect_rratio 0.208333) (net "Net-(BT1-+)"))
  (pad "2" thru_hole oval (at 2 0 270) (size 1.2 1.75) (drill 0.75) (layers "*.Cu" "*.Mask") (remove_unused_layers no) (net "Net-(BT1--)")))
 (gr_rect (start 101.805 49.08) (end 126.805 84.08) (radius 2) (stroke (width 0.05) (type solid)) (fill no) (layer "Edge.Cuts"))
 (segment (start 123.2 53.7) (end 124.75 53.7) (width 0.2) (layer "F.Cu") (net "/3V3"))
 (segment (start 123.2 54.65741) (end 123.2 53.7) (width 0.2) (layer "F.Cu") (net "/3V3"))
 (segment (start 122.73241 55.125) (end 123.2 54.65741) (width 0.2) (layer "F.Cu") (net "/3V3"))
 (segment (start 124.75 53.7) (end 125.5 52.95) (width 0.2) (layer "F.Cu") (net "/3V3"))
 (segment (start 120.5 54.4) (end 120.5 54.85741) (width 0.2) (layer "F.Cu") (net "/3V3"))
 (segment (start 120.76759 55.125) (end 122.73241 55.125) (width 0.2) (layer "F.Cu") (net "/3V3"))
 (segment (start 120.5 54.85741) (end 120.76759 55.125) (width 0.2) (layer "F.Cu") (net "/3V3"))
 (segment (start 125.35 51.2) (end 125.5 51.05) (width 0.2) (layer "F.Cu") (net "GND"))
 (segment (start 123.2 51.2) (end 125.35 51.2) (width 0.2) (layer "F.Cu") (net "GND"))
 (segment (start 115.700001 53.15) (end 117.425 53.15) (width 0.2) (layer "F.Cu") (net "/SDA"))
 (segment (start 117.425 53.15) (end 118.575 52) (width 0.2) (layer "F.Cu") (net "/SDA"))
 (segment (start 118.575 52) (end 118.575 50.96759) (width 0.2) (layer "F.Cu") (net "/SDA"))
 (segment (start 118.575 50.96759) (end 119.04259 50.5) (width 0.2) (layer "F.Cu") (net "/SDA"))
 (segment (start 119.04259 50.5) (end 120 50.5) (width 0.2) (layer "F.Cu") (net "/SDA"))
 (segment (start 115.4 52.849999) (end 115.700001 53.15) (width 0.2) (layer "F.Cu") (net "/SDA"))
 (segment (start 115.4 52.6) (end 115.4 52.849999) (width 0.2) (layer "F.Cu") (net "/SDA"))
 (segment (start 120.5 50.04259) (end 120.5 50.5) (width 0.2) (layer "F.Cu") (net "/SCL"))
 (segment (start 114.6 52.6) (end 114.6 52.654506) (width 0.2) (layer "F.Cu") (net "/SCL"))
 (segment (start 114.104506 53.15) (end 113.495494 53.15) (width 0.2) (layer "F.Cu") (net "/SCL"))
 (segment (start 114.6 52.654506) (end 114.104506 53.15) (width 0.2) (layer "F.Cu") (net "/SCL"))
 (segment (start 113.17 52.824506) (end 113.17 50.775494) (width 0.2) (layer "F.Cu") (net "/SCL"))
 (segment (start 113.495494 53.15) (end 113.17 52.824506) (width 0.2) (layer "F.Cu") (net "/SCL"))
 (segment (start 120.23241 49.775) (end 120.5 50.04259) (width 0.2) (layer "F.Cu") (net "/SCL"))
 (segment (start 114.170494 49.775) (end 120.23241 49.775) (width 0.2) (layer "F.Cu") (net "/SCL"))
 (segment (start 113.17 50.775494) (end 114.170494 49.775) (width 0.2) (layer "F.Cu") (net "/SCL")))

